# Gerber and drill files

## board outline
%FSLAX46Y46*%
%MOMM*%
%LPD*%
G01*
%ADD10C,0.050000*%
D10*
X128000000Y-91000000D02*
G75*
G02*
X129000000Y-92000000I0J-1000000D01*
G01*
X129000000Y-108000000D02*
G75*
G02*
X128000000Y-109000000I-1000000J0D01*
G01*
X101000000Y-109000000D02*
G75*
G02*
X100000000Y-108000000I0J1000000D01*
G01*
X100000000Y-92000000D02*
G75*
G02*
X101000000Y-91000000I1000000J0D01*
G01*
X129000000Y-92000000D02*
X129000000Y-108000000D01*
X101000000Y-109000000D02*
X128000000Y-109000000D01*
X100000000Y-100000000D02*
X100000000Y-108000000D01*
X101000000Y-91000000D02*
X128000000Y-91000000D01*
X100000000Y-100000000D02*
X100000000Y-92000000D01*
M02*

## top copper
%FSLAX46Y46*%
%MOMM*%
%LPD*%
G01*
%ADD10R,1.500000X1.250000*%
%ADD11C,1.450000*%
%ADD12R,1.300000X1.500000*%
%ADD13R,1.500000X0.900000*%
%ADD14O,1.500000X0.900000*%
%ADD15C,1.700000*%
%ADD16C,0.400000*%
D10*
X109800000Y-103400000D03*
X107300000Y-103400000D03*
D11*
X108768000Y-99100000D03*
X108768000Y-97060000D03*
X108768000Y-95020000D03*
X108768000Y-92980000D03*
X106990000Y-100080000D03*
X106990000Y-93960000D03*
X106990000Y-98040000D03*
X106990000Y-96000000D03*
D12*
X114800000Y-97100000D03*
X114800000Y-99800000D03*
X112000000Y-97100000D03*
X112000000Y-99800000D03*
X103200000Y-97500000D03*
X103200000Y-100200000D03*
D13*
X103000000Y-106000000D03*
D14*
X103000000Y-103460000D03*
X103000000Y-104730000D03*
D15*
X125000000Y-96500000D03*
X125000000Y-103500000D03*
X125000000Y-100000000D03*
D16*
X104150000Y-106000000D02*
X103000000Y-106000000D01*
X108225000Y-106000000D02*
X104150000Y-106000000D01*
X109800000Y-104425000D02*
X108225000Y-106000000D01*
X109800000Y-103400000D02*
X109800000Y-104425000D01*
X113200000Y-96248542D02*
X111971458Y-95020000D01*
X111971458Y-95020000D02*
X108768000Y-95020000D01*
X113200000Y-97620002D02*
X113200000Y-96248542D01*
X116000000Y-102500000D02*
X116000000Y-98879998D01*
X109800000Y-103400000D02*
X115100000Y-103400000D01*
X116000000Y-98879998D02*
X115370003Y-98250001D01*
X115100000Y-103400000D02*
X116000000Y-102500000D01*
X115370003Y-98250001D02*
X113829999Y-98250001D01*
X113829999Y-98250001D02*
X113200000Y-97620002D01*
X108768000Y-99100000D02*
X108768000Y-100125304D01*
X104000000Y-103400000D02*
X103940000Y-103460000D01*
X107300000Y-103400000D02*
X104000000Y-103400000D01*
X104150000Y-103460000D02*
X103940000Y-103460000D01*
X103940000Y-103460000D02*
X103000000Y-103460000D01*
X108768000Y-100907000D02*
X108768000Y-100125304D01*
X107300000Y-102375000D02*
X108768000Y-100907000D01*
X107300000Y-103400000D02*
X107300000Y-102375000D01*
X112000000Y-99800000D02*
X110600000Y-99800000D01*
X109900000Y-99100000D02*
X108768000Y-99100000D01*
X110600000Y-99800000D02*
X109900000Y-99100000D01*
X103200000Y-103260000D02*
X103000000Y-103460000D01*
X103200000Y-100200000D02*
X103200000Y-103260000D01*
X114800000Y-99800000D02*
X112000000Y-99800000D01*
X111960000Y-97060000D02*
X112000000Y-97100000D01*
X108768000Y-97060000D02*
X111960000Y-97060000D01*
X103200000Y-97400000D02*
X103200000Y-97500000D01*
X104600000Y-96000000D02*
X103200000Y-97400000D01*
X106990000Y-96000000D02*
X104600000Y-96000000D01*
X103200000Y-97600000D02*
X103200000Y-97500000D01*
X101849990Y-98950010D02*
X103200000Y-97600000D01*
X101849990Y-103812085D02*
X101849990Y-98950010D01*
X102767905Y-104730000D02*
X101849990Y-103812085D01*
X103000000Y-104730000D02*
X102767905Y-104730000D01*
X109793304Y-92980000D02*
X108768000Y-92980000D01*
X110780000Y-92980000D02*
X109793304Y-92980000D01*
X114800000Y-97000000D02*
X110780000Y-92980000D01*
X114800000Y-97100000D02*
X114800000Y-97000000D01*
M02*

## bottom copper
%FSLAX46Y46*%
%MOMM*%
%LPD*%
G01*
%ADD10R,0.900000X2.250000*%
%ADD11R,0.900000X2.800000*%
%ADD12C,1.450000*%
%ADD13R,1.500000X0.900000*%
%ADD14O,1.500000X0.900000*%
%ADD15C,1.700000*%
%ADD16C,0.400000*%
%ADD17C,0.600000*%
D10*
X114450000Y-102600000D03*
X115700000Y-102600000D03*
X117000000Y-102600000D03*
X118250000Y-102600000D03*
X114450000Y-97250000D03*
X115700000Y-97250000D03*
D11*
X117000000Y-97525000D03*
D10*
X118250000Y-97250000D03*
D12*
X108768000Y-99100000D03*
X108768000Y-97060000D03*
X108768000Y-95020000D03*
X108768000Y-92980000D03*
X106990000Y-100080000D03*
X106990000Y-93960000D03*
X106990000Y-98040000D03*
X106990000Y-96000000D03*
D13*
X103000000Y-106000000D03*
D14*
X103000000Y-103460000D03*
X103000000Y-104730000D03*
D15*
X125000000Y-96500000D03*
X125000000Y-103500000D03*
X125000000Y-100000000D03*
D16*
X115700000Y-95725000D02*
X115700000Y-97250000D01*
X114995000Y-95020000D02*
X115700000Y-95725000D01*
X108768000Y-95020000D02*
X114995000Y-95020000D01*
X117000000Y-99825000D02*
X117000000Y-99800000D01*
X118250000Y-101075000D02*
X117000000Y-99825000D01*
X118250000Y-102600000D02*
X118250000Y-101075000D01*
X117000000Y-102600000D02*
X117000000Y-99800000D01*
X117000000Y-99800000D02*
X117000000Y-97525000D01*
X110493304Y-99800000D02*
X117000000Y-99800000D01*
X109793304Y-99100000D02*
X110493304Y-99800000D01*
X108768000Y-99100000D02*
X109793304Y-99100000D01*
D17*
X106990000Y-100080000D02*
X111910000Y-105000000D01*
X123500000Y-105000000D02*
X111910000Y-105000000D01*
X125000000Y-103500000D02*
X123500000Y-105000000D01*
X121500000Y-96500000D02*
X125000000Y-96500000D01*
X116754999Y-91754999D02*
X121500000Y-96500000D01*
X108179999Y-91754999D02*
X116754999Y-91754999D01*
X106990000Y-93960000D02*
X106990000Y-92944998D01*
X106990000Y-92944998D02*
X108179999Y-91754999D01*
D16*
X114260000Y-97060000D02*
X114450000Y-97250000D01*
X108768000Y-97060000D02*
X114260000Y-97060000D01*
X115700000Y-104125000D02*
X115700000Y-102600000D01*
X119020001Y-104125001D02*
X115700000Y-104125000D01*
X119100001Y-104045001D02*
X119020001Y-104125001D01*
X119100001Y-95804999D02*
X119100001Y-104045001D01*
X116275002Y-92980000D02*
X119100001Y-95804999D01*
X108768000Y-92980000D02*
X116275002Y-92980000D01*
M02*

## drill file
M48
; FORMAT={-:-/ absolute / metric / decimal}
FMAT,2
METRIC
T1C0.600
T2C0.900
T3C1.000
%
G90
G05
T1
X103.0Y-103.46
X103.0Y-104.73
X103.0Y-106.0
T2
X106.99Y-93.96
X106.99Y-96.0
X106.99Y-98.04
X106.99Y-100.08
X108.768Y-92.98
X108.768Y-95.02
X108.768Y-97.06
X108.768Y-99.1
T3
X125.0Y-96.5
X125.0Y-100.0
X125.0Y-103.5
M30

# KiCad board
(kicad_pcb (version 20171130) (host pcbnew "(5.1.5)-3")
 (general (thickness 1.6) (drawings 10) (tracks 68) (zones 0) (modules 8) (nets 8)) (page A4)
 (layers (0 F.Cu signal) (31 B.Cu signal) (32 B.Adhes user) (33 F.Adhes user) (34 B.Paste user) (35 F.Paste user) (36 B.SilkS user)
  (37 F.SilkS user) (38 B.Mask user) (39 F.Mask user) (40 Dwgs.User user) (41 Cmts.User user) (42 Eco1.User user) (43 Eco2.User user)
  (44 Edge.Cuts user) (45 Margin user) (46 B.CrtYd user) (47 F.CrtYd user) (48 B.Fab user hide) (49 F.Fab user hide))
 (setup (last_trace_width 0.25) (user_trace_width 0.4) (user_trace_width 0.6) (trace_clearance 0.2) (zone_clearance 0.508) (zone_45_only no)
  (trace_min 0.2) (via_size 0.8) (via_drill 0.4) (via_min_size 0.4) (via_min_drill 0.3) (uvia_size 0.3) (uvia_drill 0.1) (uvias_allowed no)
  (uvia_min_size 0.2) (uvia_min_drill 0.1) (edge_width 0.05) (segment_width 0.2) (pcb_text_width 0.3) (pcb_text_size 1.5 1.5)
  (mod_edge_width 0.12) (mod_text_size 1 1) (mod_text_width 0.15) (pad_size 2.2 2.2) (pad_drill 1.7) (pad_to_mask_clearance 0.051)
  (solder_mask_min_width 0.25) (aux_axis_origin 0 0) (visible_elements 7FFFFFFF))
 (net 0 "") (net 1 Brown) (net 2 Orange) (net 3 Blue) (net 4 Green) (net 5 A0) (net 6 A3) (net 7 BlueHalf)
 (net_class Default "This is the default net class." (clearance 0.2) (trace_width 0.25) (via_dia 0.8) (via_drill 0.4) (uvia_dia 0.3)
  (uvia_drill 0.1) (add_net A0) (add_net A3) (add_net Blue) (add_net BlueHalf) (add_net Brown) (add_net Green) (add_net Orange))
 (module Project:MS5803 (layer B.Cu) (at 116.35 100 90)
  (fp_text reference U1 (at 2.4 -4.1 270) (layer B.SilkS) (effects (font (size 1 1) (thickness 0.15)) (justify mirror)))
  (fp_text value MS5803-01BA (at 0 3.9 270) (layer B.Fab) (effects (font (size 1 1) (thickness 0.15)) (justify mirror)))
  (pad 8 smd rect (at -2.6 -1.9 90) (size 2.25 0.9) (layers B.Cu B.Paste B.Mask) (solder_mask_margin 0.1))
  (pad 7 smd rect (at -2.6 -0.65 90) (size 2.25 0.9) (layers B.Cu B.Paste B.Mask) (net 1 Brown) (solder_mask_margin 0.1))
  (pad 6 smd rect (at -2.6 0.65 90) (size 2.25 0.9) (layers B.Cu B.Paste B.Mask) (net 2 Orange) (solder_mask_margin 0.1))
  (pad 5 smd rect (at -2.6 1.9 90) (size 2.25 0.9) (layers B.Cu B.Paste B.Mask) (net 2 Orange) (solder_mask_margin 0.1))
  (pad 1 smd rect (at 2.75 -1.9 90) (size 2.25 0.9) (layers B.Cu B.Paste B.Mask) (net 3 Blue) (solder_mask_margin 0.1))
  (pad 2 smd rect (at 2.75 -0.65 90) (size 2.25 0.9) (layers B.Cu B.Paste B.Mask) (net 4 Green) (solder_mask_margin 0.1))
  (pad 3 smd rect (at 2.475 0.65 90) (size 2.8 0.9) (layers B.Cu B.Paste B.Mask) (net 2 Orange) (solder_mask_margin 0.1))
  (pad 4 smd rect (at 2.75 1.9 90) (size 2.25 0.9) (layers B.Cu B.Paste B.Mask) (solder_mask_margin 0.1)))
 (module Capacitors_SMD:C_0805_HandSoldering (layer F.Cu) (at 108.55 103.4)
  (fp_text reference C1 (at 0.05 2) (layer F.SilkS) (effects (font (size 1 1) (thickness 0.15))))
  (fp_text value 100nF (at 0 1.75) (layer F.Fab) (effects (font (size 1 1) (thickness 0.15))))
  (pad 2 smd rect (at 1.25 0) (size 1.5 1.25) (layers F.Cu F.Paste F.Mask) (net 4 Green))
  (pad 1 smd rect (at -1.25 0) (size 1.5 1.25) (layers F.Cu F.Paste F.Mask) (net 2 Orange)))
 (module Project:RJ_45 (layer F.Cu) (at 107 100.09 270)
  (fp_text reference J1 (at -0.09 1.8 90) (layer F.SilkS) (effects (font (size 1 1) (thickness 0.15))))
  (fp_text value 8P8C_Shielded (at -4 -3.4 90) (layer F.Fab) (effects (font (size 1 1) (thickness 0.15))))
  (pad 2 thru_hole circle (at -0.99 -1.768 270) (size 1.45 1.45) (drill 0.9) (layers *.Cu *.Mask) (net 2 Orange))
  (pad 4 thru_hole circle (at -3.03 -1.768 270) (size 1.45 1.45) (drill 0.9) (layers *.Cu *.Mask) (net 3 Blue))
  (pad 6 thru_hole circle (at -5.07 -1.768 270) (size 1.45 1.45) (drill 0.9) (layers *.Cu *.Mask) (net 4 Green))
  (pad 8 thru_hole circle (at -7.11 -1.768 270) (size 1.45 1.45) (drill 0.9) (layers *.Cu *.Mask) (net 1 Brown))
  (pad 1 thru_hole circle (at -0.01 0.01 270) (size 1.45 1.45) (drill 0.9) (layers *.Cu *.Mask) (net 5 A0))
  (pad 7 thru_hole circle (at -6.13 0.01 270) (size 1.45 1.45) (drill 0.9) (layers *.Cu *.Mask) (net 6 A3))
  (pad 3 thru_hole circle (at -2.05 0.01 270) (size 1.45 1.45) (drill 0.9) (layers *.Cu *.Mask))
  (pad 5 thru_hole circle (at -4.09 0.01 270) (size 1.45 1.45) (drill 0.9) (layers *.Cu *.Mask) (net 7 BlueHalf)))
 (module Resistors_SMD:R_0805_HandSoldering (layer F.Cu) (at 114.8 98.45 90)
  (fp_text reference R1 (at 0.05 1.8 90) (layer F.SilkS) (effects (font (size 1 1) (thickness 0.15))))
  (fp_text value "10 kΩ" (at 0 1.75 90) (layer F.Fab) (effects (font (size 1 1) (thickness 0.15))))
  (pad 2 smd rect (at 1.35 0 90) (size 1.5 1.3) (layers F.Cu F.Paste F.Mask) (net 1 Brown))
  (pad 1 smd rect (at -1.35 0 90) (size 1.5 1.3) (layers F.Cu F.Paste F.Mask) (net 2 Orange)))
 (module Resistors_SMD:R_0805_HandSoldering (layer F.Cu) (at 112 98.45 270)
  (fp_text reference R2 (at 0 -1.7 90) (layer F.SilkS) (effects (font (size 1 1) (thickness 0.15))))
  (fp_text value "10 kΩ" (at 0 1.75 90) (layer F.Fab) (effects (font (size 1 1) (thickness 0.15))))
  (pad 1 smd rect (at -1.35 0 270) (size 1.5 1.3) (layers F.Cu F.Paste F.Mask) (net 3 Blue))
  (pad 2 smd rect (at 1.35 0 270) (size 1.5 1.3) (layers F.Cu F.Paste F.Mask) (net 2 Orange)))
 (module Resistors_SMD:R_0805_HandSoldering (layer F.Cu) (at 103.2 98.85 90)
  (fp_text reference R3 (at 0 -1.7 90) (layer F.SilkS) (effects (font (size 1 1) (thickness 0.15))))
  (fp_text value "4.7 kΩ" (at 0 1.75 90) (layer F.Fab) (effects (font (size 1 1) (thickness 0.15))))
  (pad 2 smd rect (at 1.35 0 90) (size 1.5 1.3) (layers F.Cu F.Paste F.Mask) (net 7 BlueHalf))
  (pad 1 smd rect (at -1.35 0 90) (size 1.5 1.3) (layers F.Cu F.Paste F.Mask) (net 2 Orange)))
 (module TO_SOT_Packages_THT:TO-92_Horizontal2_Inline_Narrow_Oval (layer F.Cu) (at 103 106 90)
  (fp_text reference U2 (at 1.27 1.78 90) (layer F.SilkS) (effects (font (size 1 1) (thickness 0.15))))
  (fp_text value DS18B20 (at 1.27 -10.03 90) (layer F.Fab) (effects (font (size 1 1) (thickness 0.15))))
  (pad 1 thru_hole rect (at 0 0 270) (size 0.9 1.5) (drill 0.6) (layers *.Cu *.Mask) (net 4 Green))
  (pad 3 thru_hole oval (at 2.54 0 270) (size 0.9 1.5) (drill 0.6) (layers *.Cu *.Mask) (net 2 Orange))
  (pad 2 thru_hole oval (at 1.27 0 270) (size 0.9 1.5) (drill 0.6) (layers *.Cu *.Mask) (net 7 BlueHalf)))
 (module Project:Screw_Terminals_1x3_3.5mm (layer F.Cu) (at 125 103.5 90)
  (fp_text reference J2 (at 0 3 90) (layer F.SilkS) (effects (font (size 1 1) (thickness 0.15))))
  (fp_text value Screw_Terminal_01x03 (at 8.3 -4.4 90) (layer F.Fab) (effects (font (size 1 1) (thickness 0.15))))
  (pad 3 thru_hole circle (at 7 0 90) (size 1.7 1.7) (drill 1) (layers *.Cu *.Mask) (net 6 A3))
  (pad 1 thru_hole circle (at 0 0 90) (size 1.7 1.7) (drill 1) (layers *.Cu *.Mask) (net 5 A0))
  (pad 2 thru_hole circle (at 3.5 0 90) (size 1.7 1.7) (drill 1) (layers *.Cu *.Mask)))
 (gr_arc (start 128 92) (end 129 92) (angle -90) (layer Edge.Cuts) (width 0.05))
 (gr_arc (start 128 108) (end 128 109) (angle -90) (layer Edge.Cuts) (width 0.05))
 (gr_arc (start 101 108) (end 100 108) (angle -90) (layer Edge.Cuts) (width 0.05))
 (gr_arc (start 101 92) (end 101 91) (angle -90) (layer Edge.Cuts) (width 0.05))
 (gr_line (start 129 92) (end 129 108) (layer Edge.Cuts) (width 0.05))
 (gr_line (start 101 109) (end 128 109) (layer Edge.Cuts) (width 0.05))
 (gr_line (start 100 100) (end 100 108) (layer Edge.Cuts) (width 0.05))
 (gr_line (start 101 91) (end 128 91) (layer Edge.Cuts) (width 0.05))
 (gr_line (start 100 100) (end 100 92) (layer Edge.Cuts) (width 0.05))
 (segment (start 115.7 95.725) (end 115.7 97.25) (width 0.4) (layer B.Cu) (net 4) (status 20))
 (segment (start 114.995 95.02) (end 115.7 95.725) (width 0.4) (layer B.Cu) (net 4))
 (segment (start 108.768 95.02) (end 114.995 95.02) (width 0.4) (layer B.Cu) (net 4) (status 10))
 (segment (start 104.15 106) (end 103 106) (width 0.4) (layer F.Cu) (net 4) (status 20))
 (segment (start 108.225 106) (end 104.15 106) (width 0.4) (layer F.Cu) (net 4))
 (segment (start 109.8 104.425) (end 108.225 106) (width 0.4) (layer F.Cu) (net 4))
 (segment (start 109.8 103.4) (end 109.8 104.425) (width 0.4) (layer F.Cu) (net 4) (status 10))
 (segment (start 113.2 96.248542) (end 111.971458 95.02) (width 0.4) (layer F.Cu) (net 4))
 (segment (start 111.971458 95.02) (end 108.768 95.02) (width 0.4) (layer F.Cu) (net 4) (status 20))
 (segment (start 113.2 97.620002) (end 113.2 96.248542) (width 0.4) (layer F.Cu) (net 4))
 (segment (start 116 102.5) (end 116 98.879998) (width 0.4) (layer F.Cu) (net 4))
 (segment (start 109.8 103.4) (end 115.1 103.4) (width 0.4) (layer F.Cu) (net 4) (status 10))
 (segment (start 116 98.879998) (end 115.370003 98.250001) (width 0.4) (layer F.Cu) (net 4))
 (segment (start 115.1 103.4) (end 116 102.5) (width 0.4) (layer F.Cu) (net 4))
 (segment (start 115.370003 98.250001) (end 113.829999 98.250001) (width 0.4) (layer F.Cu) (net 4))
 (segment (start 113.829999 98.250001) (end 113.2 97.620002) (width 0.4) (layer F.Cu) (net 4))
 (segment (start 117 99.825) (end 117 99.8) (width 0.4) (layer B.Cu) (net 2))
 (segment (start 118.25 101.075) (end 117 99.825) (width 0.4) (layer B.Cu) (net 2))
 (segment (start 118.25 102.6) (end 118.25 101.075) (width 0.4) (layer B.Cu) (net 2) (status 10))
 (segment (start 117 102.6) (end 117 99.8) (width 0.4) (layer B.Cu) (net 2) (status 10))
 (segment (start 117 99.8) (end 117 97.525) (width 0.4) (layer B.Cu) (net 2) (status 20))
 (segment (start 110.493304 99.8) (end 117 99.8) (width 0.4) (layer B.Cu) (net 2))
 (segment (start 109.793304 99.1) (end 110.493304 99.8) (width 0.4) (layer B.Cu) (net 2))
 (segment (start 108.768 99.1) (end 109.793304 99.1) (width 0.4) (layer B.Cu) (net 2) (status 10))
 (segment (start 108.768 99.1) (end 108.768 100.125304) (width 0.4) (layer F.Cu) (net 2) (status 10))
 (segment (start 104 103.4) (end 103.94 103.46) (width 0.4) (layer F.Cu) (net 2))
 (segment (start 107.3 103.4) (end 104 103.4) (width 0.4) (layer F.Cu) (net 2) (status 10))
 (segment (start 104.15 103.46) (end 103.94 103.46) (width 0.4) (layer F.Cu) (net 2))
 (segment (start 103.94 103.46) (end 103 103.46) (width 0.4) (layer F.Cu) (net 2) (status 20))
 (segment (start 108.768 100.907) (end 108.768 100.125304) (width 0.4) (layer F.Cu) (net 2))
 (segment (start 107.3 102.375) (end 108.768 100.907) (width 0.4) (layer F.Cu) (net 2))
 (segment (start 107.3 103.4) (end 107.3 102.375) (width 0.4) (layer F.Cu) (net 2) (status 10))
 (segment (start 112 99.8) (end 110.6 99.8) (width 0.4) (layer F.Cu) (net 2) (status 10))
 (segment (start 109.9 99.1) (end 108.768 99.1) (width 0.4) (layer F.Cu) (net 2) (status 20))
 (segment (start 110.6 99.8) (end 109.9 99.1) (width 0.4) (layer F.Cu) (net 2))
 (segment (start 103.2 103.26) (end 103 103.46) (width 0.4) (layer F.Cu) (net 2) (status 30))
 (segment (start 103.2 100.2) (end 103.2 103.26) (width 0.4) (layer F.Cu) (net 2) (status 30))
 (segment (start 114.8 99.8) (end 112 99.8) (width 0.4) (layer F.Cu) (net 2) (status 30))
 (segment (start 106.99 100.08) (end 111.91 105) (width 0.6) (layer B.Cu) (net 5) (status 10))
 (segment (start 123.5 105) (end 111.91 105) (width 0.6) (layer B.Cu) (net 5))
 (segment (start 125 103.5) (end 123.5 105) (width 0.6) (layer B.Cu) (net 5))
 (segment (start 121.5 96.5) (end 125 96.5) (width 0.6) (layer B.Cu) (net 6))
 (segment (start 116.754999 91.754999) (end 121.5 96.5) (width 0.6) (layer B.Cu) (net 6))
 (segment (start 108.179999 91.754999) (end 116.754999 91.754999) (width 0.6) (layer B.Cu) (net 6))
 (segment (start 106.99 93.96) (end 106.99 92.944998) (width 0.6) (layer B.Cu) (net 6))
 (segment (start 106.99 92.944998) (end 108.179999 91.754999) (width 0.6) (layer B.Cu) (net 6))
 (segment (start 114.26 97.06) (end 114.45 97.25) (width 0.4) (layer B.Cu) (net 3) (status 30))
 (segment (start 108.768 97.06) (end 114.26 97.06) (width 0.4) (layer B.Cu) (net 3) (status 30))
 (segment (start 111.96 97.06) (end 112 97.1) (width 0.4) (layer F.Cu) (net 3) (status 30))
 (segment (start 108.768 97.06) (end 111.96 97.06) (width 0.4) (layer F.Cu) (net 3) (status 30))
 (segment (start 103.2 97.4) (end 103.2 97.5) (width 0.4) (layer F.Cu) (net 7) (status 30))
 (segment (start 104.6 96) (end 103.2 97.4) (width 0.4) (layer F.Cu) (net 7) (status 20))
 (segment (start 106.99 96) (end 104.6 96) (width 0.4) (layer F.Cu) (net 7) (status 10))
 (segment (start 103.2 97.6) (end 103.2 97.5) (width 0.4) (layer F.Cu) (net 7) (status 30))
 (segment (start 101.84999 98.95001) (end 103.2 97.6) (width 0.4) (layer F.Cu) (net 7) (status 20))
 (segment (start 101.84999 103.812085) (end 101.84999 98.95001) (width 0.4) (layer F.Cu) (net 7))
 (segment (start 102.767905 104.73) (end 101.84999 103.812085) (width 0.4) (layer F.Cu) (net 7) (status 10))
 (segment (start 103 104.73) (end 102.767905 104.73) (width 0.4) (layer F.Cu) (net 7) (status 30))
 (segment (start 115.7 104.125) (end 115.7 102.6) (width 0.4) (layer B.Cu) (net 1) (status 20))
 (segment (start 119.020001 104.125001) (end 115.7 104.125) (width 0.4) (layer B.Cu) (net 1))
 (segment (start 119.100001 104.045001) (end 119.020001 104.125001) (width 0.4) (layer B.Cu) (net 1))
 (segment (start 119.100001 95.804999) (end 119.100001 104.045001) (width 0.4) (layer B.Cu) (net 1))
 (segment (start 116.275002 92.98) (end 119.100001 95.804999) (width 0.4) (layer B.Cu) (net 1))
 (segment (start 108.768 92.98) (end 116.275002 92.98) (width 0.4) (layer B.Cu) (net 1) (status 10))
 (segment (start 109.793304 92.98) (end 108.768 92.98) (width 0.4) (layer F.Cu) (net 1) (status 20))
 (segment (start 110.78 92.98) (end 109.793304 92.98) (width 0.4) (layer F.Cu) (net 1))
 (segment (start 114.8 97) (end 110.78 92.98) (width 0.4) (layer F.Cu) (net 1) (status 10))
 (segment (start 114.8 97.1) (end 114.8 97) (width 0.4) (layer F.Cu) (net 1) (status 30)))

